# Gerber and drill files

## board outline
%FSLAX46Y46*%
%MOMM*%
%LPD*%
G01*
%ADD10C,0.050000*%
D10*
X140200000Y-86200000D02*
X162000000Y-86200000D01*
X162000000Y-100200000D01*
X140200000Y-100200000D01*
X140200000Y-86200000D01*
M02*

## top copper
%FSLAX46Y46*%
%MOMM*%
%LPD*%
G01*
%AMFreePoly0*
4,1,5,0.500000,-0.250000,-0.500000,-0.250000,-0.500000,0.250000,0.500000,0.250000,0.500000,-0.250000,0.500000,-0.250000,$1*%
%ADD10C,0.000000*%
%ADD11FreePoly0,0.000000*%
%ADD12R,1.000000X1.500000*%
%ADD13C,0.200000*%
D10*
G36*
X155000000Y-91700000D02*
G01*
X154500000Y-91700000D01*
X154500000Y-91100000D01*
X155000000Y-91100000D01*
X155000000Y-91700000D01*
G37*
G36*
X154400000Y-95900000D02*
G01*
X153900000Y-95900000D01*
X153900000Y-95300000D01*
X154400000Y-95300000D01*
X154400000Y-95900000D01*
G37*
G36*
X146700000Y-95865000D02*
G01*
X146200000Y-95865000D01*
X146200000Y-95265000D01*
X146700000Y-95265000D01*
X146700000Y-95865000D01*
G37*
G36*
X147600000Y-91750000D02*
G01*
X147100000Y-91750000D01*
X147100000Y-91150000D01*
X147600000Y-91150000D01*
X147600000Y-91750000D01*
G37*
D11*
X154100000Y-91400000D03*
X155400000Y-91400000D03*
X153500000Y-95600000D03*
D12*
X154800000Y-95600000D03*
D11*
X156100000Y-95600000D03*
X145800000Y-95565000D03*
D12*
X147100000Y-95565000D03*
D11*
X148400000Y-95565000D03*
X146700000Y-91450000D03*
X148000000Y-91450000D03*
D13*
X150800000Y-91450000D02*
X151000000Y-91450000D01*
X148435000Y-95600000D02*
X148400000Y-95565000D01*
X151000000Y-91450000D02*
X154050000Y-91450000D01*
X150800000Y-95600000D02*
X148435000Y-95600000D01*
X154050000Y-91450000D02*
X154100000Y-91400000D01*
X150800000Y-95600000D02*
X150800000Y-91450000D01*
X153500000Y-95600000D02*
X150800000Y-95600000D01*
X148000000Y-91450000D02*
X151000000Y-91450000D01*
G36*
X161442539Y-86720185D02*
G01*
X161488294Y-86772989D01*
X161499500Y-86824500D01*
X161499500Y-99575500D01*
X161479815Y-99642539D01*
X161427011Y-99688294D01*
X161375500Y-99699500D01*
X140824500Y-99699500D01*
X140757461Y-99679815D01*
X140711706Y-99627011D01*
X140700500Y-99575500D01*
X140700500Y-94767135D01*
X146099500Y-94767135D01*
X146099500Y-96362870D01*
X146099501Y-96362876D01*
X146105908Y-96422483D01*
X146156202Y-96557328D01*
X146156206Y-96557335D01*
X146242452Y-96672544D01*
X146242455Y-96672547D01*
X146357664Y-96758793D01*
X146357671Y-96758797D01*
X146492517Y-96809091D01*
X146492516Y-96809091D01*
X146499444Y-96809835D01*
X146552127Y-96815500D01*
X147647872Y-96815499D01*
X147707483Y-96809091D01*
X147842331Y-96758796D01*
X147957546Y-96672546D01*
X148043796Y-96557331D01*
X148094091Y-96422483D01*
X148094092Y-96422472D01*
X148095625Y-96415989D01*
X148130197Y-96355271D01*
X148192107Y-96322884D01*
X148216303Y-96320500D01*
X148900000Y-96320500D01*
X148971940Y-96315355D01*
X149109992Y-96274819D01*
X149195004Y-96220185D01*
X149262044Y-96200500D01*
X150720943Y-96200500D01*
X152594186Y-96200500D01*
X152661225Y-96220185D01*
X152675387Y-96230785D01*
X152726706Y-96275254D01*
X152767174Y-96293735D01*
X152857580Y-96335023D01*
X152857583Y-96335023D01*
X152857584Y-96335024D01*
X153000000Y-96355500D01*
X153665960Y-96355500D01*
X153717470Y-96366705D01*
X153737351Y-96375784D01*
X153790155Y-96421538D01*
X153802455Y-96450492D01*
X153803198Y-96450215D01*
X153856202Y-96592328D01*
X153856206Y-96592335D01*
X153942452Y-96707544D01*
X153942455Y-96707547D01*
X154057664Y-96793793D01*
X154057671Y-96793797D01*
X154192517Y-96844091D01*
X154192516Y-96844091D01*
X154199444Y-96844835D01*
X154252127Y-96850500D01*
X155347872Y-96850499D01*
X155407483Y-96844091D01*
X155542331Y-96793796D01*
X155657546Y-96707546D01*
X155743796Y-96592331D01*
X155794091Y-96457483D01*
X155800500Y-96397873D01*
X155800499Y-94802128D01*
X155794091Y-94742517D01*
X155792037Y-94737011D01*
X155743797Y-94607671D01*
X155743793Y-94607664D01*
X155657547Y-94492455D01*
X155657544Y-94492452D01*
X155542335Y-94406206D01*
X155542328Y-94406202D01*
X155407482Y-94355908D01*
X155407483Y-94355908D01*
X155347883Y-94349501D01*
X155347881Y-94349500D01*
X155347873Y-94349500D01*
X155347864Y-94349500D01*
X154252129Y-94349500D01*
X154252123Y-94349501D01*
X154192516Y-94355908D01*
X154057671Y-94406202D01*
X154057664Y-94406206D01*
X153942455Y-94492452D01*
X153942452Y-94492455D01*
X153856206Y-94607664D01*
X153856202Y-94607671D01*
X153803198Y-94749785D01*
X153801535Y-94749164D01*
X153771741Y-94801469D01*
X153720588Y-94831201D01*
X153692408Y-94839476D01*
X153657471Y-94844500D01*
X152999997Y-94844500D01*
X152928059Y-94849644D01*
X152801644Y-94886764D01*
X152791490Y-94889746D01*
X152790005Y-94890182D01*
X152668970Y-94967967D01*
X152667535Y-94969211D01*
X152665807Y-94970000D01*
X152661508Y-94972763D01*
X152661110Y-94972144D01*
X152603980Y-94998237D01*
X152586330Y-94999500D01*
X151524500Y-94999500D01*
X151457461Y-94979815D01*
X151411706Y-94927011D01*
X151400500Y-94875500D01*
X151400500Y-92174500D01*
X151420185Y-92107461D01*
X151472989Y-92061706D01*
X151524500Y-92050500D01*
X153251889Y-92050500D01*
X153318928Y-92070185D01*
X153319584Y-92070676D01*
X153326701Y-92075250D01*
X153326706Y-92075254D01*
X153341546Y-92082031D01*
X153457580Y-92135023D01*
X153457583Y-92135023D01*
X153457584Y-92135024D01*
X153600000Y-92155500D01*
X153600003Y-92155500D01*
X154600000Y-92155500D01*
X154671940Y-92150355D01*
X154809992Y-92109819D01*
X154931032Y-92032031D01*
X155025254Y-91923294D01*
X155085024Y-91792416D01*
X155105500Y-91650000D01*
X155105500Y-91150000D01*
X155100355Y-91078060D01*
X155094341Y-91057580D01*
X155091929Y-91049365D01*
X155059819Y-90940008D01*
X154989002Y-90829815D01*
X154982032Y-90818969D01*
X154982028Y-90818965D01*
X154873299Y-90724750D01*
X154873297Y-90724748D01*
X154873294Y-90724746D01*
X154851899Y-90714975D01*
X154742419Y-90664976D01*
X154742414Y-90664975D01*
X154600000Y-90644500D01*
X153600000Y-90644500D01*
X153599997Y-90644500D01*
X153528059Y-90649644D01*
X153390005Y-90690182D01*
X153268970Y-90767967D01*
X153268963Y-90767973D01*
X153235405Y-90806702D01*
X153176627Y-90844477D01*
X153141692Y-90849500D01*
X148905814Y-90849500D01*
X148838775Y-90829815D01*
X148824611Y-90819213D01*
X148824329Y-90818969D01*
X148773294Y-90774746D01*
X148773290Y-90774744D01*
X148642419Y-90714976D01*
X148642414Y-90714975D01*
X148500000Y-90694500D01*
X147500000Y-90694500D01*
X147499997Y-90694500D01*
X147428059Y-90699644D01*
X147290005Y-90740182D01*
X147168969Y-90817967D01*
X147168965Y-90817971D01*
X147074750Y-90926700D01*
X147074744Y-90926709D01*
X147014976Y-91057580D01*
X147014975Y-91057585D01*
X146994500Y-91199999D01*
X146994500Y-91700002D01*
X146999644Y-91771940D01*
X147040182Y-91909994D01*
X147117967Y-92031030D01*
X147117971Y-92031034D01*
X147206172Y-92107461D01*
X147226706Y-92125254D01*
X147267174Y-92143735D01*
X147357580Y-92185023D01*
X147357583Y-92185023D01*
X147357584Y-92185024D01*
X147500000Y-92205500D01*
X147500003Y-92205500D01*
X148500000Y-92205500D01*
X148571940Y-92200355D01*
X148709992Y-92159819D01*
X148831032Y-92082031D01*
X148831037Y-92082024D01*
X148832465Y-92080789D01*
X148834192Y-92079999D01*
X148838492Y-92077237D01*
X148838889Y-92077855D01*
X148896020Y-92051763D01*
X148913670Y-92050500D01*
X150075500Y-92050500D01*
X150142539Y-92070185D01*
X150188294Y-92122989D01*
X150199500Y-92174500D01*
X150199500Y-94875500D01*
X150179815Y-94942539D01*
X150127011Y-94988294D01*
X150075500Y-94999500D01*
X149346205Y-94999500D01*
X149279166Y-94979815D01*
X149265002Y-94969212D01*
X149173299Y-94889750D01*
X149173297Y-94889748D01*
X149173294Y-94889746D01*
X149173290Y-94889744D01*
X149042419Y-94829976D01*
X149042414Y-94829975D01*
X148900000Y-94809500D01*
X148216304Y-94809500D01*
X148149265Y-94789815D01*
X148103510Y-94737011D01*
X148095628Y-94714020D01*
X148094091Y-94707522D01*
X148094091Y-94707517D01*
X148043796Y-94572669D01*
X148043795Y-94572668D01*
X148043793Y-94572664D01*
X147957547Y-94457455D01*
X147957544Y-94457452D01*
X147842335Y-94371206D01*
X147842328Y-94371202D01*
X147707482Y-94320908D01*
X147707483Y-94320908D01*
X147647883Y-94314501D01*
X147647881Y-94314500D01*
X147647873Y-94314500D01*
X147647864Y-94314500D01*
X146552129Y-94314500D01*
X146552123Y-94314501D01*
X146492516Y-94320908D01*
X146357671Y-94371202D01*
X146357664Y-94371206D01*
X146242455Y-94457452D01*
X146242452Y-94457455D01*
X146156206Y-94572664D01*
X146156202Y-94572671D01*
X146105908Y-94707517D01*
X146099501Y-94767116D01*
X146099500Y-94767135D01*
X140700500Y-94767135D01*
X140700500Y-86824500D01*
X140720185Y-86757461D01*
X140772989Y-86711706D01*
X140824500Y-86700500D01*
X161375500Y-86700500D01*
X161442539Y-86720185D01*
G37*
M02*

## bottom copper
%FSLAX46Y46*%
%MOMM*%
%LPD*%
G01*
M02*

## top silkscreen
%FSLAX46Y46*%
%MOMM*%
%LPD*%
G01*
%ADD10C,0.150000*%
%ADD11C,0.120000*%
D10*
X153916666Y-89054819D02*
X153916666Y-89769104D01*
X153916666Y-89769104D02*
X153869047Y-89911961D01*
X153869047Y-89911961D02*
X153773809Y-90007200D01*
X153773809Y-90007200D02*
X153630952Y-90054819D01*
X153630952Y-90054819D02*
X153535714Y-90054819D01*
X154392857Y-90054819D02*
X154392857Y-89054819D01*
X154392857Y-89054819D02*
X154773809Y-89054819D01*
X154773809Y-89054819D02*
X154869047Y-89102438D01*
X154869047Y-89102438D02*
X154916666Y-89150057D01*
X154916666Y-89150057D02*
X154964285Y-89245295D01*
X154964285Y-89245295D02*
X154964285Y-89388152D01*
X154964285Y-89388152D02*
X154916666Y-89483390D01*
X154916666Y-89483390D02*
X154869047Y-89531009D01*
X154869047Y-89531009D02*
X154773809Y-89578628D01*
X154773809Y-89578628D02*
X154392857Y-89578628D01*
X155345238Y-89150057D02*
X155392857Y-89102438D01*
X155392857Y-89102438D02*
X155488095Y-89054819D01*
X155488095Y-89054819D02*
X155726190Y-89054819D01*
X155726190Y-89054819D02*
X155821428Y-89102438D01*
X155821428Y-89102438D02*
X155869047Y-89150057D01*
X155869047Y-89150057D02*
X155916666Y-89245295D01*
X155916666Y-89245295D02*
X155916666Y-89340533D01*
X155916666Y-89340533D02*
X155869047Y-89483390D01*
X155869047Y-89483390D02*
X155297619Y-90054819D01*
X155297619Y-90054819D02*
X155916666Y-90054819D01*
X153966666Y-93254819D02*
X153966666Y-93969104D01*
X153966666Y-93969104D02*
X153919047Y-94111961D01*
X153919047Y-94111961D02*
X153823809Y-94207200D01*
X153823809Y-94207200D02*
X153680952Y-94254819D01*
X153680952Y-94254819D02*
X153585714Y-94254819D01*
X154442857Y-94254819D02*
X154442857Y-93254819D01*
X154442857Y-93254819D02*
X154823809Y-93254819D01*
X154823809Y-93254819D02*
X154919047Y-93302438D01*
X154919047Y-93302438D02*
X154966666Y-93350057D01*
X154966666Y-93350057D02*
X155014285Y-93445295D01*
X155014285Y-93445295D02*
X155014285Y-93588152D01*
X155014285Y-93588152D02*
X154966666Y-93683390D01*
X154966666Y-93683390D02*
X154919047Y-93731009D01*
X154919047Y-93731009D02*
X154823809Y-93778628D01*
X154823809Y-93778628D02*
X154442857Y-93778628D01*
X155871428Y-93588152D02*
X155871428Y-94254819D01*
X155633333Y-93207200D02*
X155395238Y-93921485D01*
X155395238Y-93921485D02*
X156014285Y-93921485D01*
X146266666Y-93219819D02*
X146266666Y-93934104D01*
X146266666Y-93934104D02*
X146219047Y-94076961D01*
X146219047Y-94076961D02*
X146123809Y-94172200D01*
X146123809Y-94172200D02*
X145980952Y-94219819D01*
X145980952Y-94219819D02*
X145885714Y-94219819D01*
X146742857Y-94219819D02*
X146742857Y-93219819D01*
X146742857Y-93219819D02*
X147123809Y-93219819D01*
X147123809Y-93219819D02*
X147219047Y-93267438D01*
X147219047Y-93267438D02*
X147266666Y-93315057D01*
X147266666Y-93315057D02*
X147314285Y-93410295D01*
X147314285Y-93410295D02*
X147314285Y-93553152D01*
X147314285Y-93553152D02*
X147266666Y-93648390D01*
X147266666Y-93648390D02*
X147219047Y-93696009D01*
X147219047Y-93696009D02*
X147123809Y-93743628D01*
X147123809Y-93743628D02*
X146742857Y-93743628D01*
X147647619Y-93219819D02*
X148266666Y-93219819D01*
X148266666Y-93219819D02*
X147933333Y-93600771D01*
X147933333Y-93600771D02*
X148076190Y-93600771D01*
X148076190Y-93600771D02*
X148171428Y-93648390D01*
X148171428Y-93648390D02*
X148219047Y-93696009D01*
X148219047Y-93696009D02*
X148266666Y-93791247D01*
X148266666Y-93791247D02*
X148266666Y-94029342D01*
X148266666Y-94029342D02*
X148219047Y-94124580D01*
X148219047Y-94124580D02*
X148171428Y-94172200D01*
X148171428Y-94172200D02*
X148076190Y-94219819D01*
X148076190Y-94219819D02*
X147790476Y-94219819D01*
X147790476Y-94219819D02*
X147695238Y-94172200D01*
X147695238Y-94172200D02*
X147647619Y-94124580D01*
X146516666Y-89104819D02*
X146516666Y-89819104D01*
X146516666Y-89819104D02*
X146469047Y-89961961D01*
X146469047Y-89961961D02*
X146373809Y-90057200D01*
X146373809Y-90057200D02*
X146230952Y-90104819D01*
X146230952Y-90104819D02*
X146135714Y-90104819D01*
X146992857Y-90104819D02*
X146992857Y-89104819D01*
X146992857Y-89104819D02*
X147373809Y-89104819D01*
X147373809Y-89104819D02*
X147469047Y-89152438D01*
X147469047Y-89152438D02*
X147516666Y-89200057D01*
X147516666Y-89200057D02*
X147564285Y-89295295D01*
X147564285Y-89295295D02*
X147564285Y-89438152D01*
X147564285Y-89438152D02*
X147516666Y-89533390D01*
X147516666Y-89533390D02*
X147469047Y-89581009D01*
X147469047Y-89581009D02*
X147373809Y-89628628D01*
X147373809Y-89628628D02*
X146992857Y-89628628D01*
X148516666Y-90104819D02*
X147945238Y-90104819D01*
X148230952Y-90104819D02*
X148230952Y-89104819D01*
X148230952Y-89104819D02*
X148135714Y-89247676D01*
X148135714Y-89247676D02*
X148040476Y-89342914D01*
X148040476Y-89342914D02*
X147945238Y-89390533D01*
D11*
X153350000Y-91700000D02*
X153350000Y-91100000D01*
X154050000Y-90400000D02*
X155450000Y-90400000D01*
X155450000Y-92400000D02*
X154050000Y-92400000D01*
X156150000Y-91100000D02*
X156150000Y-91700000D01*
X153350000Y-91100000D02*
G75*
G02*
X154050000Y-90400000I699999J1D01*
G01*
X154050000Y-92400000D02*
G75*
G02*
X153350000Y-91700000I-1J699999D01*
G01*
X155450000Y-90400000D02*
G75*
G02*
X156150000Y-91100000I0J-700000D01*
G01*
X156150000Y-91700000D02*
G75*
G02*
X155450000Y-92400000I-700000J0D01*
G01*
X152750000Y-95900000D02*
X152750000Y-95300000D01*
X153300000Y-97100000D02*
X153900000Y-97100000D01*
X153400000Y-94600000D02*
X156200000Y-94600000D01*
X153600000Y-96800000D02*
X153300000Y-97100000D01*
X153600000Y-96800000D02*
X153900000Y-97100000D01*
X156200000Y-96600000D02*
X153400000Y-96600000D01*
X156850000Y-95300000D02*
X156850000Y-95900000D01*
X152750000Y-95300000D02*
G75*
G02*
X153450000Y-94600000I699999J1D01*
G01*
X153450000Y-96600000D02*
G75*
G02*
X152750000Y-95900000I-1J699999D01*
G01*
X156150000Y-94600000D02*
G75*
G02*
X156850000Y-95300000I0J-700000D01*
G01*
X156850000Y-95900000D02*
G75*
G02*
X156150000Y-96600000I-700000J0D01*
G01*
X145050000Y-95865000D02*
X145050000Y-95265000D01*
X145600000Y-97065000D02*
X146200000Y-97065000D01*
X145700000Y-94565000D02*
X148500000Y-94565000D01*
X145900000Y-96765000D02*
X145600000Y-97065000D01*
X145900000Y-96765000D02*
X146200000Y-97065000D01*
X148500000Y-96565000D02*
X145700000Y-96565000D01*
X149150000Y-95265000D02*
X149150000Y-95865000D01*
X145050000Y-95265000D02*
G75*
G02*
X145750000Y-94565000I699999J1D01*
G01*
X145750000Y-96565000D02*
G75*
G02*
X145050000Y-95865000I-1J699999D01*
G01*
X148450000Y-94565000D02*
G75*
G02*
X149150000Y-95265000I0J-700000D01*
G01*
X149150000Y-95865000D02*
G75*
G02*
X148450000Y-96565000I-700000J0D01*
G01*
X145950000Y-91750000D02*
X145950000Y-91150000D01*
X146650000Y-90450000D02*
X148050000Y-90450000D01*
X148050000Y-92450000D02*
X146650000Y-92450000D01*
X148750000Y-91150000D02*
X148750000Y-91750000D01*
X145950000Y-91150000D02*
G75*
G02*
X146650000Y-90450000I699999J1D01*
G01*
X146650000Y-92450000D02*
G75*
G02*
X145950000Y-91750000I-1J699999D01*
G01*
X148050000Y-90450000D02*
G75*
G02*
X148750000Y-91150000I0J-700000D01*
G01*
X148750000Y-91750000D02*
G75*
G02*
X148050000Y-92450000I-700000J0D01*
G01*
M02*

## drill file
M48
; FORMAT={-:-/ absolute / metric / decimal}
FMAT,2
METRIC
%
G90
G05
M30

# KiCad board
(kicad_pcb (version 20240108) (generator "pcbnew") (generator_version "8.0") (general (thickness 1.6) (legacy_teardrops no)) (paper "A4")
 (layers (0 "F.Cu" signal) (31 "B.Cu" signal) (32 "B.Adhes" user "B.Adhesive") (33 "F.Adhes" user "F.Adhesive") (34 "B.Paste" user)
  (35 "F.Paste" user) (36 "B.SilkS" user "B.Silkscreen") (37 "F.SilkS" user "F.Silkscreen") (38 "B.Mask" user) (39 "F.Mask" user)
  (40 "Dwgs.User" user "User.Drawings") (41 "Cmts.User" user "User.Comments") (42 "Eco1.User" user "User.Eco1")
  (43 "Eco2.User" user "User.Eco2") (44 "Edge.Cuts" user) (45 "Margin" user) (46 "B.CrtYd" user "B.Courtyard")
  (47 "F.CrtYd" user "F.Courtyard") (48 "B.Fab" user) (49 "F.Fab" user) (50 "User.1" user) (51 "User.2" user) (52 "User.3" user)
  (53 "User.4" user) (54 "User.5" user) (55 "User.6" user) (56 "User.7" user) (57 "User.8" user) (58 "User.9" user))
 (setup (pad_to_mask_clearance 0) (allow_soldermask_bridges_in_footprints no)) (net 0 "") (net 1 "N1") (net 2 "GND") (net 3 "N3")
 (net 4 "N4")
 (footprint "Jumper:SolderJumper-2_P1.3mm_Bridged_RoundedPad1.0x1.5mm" (layer "F.Cu") (at 154.75 91.4)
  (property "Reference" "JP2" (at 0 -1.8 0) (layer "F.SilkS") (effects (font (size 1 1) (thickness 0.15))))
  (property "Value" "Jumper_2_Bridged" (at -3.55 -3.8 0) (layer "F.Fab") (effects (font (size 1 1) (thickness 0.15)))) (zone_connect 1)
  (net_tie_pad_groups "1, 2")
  (fp_poly (pts (xy 0.25 -0.3) (xy -0.25 -0.3) (xy -0.25 0.3) (xy 0.25 0.3)) (stroke (width 0) (type solid)) (fill solid) (layer "F.Cu"))
  (fp_line (start -1.4 0.3) (end -1.4 -0.3) (stroke (width 0.12) (type solid)) (layer "F.SilkS"))
  (fp_line (start -0.7 -1) (end 0.7 -1) (stroke (width 0.12) (type solid)) (layer "F.SilkS"))
  (fp_line (start 0.7 1) (end -0.7 1) (stroke (width 0.12) (type solid)) (layer "F.SilkS"))
  (fp_line (start 1.4 -0.3) (end 1.4 0.3) (stroke (width 0.12) (type solid)) (layer "F.SilkS"))
  (fp_arc (start -1.4 -0.3) (mid -1.194975 -0.794975) (end -0.7 -1) (stroke (width 0.12) (type solid)) (layer "F.SilkS"))
  (fp_arc (start -0.7 1) (mid -1.194975 0.794975) (end -1.4 0.3) (stroke (width 0.12) (type solid)) (layer "F.SilkS"))
  (fp_arc (start 0.7 -1) (mid 1.194975 -0.794975) (end 1.4 -0.3) (stroke (width 0.12) (type solid)) (layer "F.SilkS"))
  (fp_arc (start 1.4 0.3) (mid 1.194975 0.794975) (end 0.7 1) (stroke (width 0.12) (type solid)) (layer "F.SilkS"))
  (pad "1" smd custom (at -0.65 0) (size 1 0.5) (layers "F.Cu" "F.Mask") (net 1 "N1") (zone_connect 2) (thermal_bridge_angle 45)
   (options (clearance outline) (anchor rect)) (primitives))
  (pad "2" smd custom (at 0.65 0) (size 1 0.5) (layers "F.Cu" "F.Mask") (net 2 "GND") (zone_connect 2) (thermal_bridge_angle 45)
   (options (clearance outline) (anchor rect)) (primitives)))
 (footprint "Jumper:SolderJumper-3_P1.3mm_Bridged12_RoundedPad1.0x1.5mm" (layer "F.Cu") (at 154.8 95.6)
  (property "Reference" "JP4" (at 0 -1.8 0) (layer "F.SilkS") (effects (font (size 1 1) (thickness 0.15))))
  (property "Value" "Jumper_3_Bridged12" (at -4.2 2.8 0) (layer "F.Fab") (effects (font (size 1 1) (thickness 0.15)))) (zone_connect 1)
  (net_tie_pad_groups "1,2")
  (fp_poly (pts (xy -0.9 -0.3) (xy -0.4 -0.3) (xy -0.4 0.3) (xy -0.9 0.3)) (stroke (width 0) (type solid)) (fill solid) (layer "F.Cu"))
  (fp_line (start -2.05 0.3) (end -2.05 -0.3) (stroke (width 0.12) (type solid)) (layer "F.SilkS"))
  (fp_line (start -1.5 1.5) (end -0.9 1.5) (stroke (width 0.12) (type solid)) (layer "F.SilkS"))
  (fp_line (start -1.4 -1) (end 1.4 -1) (stroke (width 0.12) (type solid)) (layer "F.SilkS"))
  (fp_line (start -1.2 1.2) (end -1.5 1.5) (stroke (width 0.12) (type solid)) (layer "F.SilkS"))
  (fp_line (start -1.2 1.2) (end -0.9 1.5) (stroke (width 0.12) (type solid)) (layer "F.SilkS"))
  (fp_line (start 1.4 1) (end -1.4 1) (stroke (width 0.12) (type solid)) (layer "F.SilkS"))
  (fp_line (start 2.05 -0.3) (end 2.05 0.3) (stroke (width 0.12) (type solid)) (layer "F.SilkS"))
  (fp_arc (start -2.05 -0.3) (mid -1.844975 -0.794975) (end -1.35 -1) (stroke (width 0.12) (type solid)) (layer "F.SilkS"))
  (fp_arc (start -1.35 1) (mid -1.844975 0.794975) (end -2.05 0.3) (stroke (width 0.12) (type solid)) (layer "F.SilkS"))
  (fp_arc (start 1.35 -1) (mid 1.844975 -0.794975) (end 2.05 -0.3) (stroke (width 0.12) (type solid)) (layer "F.SilkS"))
  (fp_arc (start 2.05 0.3) (mid 1.844975 0.794975) (end 1.35 1) (stroke (width 0.12) (type solid)) (layer "F.SilkS"))
  (pad "1" smd custom (at -1.3 0) (size 1 0.5) (layers "F.Cu" "F.Mask") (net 1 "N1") (zone_connect 2) (thermal_bridge_angle 45)
   (options (clearance outline) (anchor rect)) (primitives))
  (pad "2" smd rect (at 0 0) (size 1 1.5) (layers "F.Cu" "F.Mask") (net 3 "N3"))
  (pad "3" smd custom (at 1.3 0) (size 1 0.5) (layers "F.Cu" "F.Mask") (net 2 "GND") (zone_connect 2) (thermal_bridge_angle 45)
   (options (clearance outline) (anchor rect)) (primitives)))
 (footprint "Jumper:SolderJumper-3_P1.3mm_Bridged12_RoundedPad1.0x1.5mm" (layer "F.Cu") (at 147.1 95.565)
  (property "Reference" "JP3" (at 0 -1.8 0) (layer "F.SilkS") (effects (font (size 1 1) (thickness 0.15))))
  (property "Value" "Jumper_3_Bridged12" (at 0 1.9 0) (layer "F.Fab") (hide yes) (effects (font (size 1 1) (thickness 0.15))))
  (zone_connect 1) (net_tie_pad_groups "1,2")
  (fp_poly (pts (xy -0.9 -0.3) (xy -0.4 -0.3) (xy -0.4 0.3) (xy -0.9 0.3)) (stroke (width 0) (type solid)) (fill solid) (layer "F.Cu"))
  (fp_line (start -2.05 0.3) (end -2.05 -0.3) (stroke (width 0.12) (type solid)) (layer "F.SilkS"))
  (fp_line (start -1.5 1.5) (end -0.9 1.5) (stroke (width 0.12) (type solid)) (layer "F.SilkS"))
  (fp_line (start -1.4 -1) (end 1.4 -1) (stroke (width 0.12) (type solid)) (layer "F.SilkS"))
  (fp_line (start -1.2 1.2) (end -1.5 1.5) (stroke (width 0.12) (type solid)) (layer "F.SilkS"))
  (fp_line (start -1.2 1.2) (end -0.9 1.5) (stroke (width 0.12) (type solid)) (layer "F.SilkS"))
  (fp_line (start 1.4 1) (end -1.4 1) (stroke (width 0.12) (type solid)) (layer "F.SilkS"))
  (fp_line (start 2.05 -0.3) (end 2.05 0.3) (stroke (width 0.12) (type solid)) (layer "F.SilkS"))
  (fp_arc (start -2.05 -0.3) (mid -1.844975 -0.794975) (end -1.35 -1) (stroke (width 0.12) (type solid)) (layer "F.SilkS"))
  (fp_arc (start -1.35 1) (mid -1.844975 0.794975) (end -2.05 0.3) (stroke (width 0.12) (type solid)) (layer "F.SilkS"))
  (fp_arc (start 1.35 -1) (mid 1.844975 -0.794975) (end 2.05 -0.3) (stroke (width 0.12) (type solid)) (layer "F.SilkS"))
  (fp_arc (start 2.05 0.3) (mid 1.844975 0.794975) (end 1.35 1) (stroke (width 0.12) (type solid)) (layer "F.SilkS"))
  (pad "1" smd custom (at -1.3 0) (size 1 0.5) (layers "F.Cu" "F.Mask") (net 2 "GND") (zone_connect 2) (thermal_bridge_angle 45)
   (options (clearance outline) (anchor rect)) (primitives))
  (pad "2" smd rect (at 0 0) (size 1 1.5) (layers "F.Cu" "F.Mask") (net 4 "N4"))
  (pad "3" smd custom (at 1.3 0) (size 1 0.5) (layers "F.Cu" "F.Mask") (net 1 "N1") (zone_connect 2) (thermal_bridge_angle 45)
   (options (clearance outline) (anchor rect)) (primitives)))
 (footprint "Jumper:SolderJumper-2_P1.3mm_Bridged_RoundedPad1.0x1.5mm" (layer "F.Cu") (at 147.35 91.45)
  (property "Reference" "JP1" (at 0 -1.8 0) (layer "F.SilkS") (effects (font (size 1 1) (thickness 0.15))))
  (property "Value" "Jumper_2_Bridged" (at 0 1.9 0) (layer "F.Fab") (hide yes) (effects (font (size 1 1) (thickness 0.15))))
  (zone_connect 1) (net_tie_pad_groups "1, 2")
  (fp_poly (pts (xy 0.25 -0.3) (xy -0.25 -0.3) (xy -0.25 0.3) (xy 0.25 0.3)) (stroke (width 0) (type solid)) (fill solid) (layer "F.Cu"))
  (fp_line (start -1.4 0.3) (end -1.4 -0.3) (stroke (width 0.12) (type solid)) (layer "F.SilkS"))
  (fp_line (start -0.7 -1) (end 0.7 -1) (stroke (width 0.12) (type solid)) (layer "F.SilkS"))
  (fp_line (start 0.7 1) (end -0.7 1) (stroke (width 0.12) (type solid)) (layer "F.SilkS"))
  (fp_line (start 1.4 -0.3) (end 1.4 0.3) (stroke (width 0.12) (type solid)) (layer "F.SilkS"))
  (fp_arc (start -1.4 -0.3) (mid -1.194975 -0.794975) (end -0.7 -1) (stroke (width 0.12) (type solid)) (layer "F.SilkS"))
  (fp_arc (start -0.7 1) (mid -1.194975 0.794975) (end -1.4 0.3) (stroke (width 0.12) (type solid)) (layer "F.SilkS"))
  (fp_arc (start 0.7 -1) (mid 1.194975 -0.794975) (end 1.4 -0.3) (stroke (width 0.12) (type solid)) (layer "F.SilkS"))
  (fp_arc (start 1.4 0.3) (mid 1.194975 0.794975) (end 0.7 1) (stroke (width 0.12) (type solid)) (layer "F.SilkS"))
  (pad "1" smd custom (at -0.65 0) (size 1 0.5) (layers "F.Cu" "F.Mask") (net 2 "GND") (zone_connect 2) (thermal_bridge_angle 45)
   (options (clearance outline) (anchor rect)) (primitives))
  (pad "2" smd custom (at 0.65 0) (size 1 0.5) (layers "F.Cu" "F.Mask") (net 1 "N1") (zone_connect 2) (thermal_bridge_angle 45)
   (options (clearance outline) (anchor rect)) (primitives)))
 (gr_rect (start 140.2 86.2) (end 162 100.2) (stroke (width 0.05) (type default)) (fill none) (layer "Edge.Cuts"))
 (segment (start 150.8 91.45) (end 151 91.45) (width 0.2) (layer "F.Cu") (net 1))
 (segment (start 148.435 95.6) (end 148.4 95.565) (width 0.2) (layer "F.Cu") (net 1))
 (segment (start 151 91.45) (end 154.05 91.45) (width 0.2) (layer "F.Cu") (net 1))
 (segment (start 150.8 95.6) (end 148.435 95.6) (width 0.2) (layer "F.Cu") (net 1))
 (segment (start 154.05 91.45) (end 154.1 91.4) (width 0.2) (layer "F.Cu") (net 1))
 (segment (start 150.8 95.6) (end 150.8 91.45) (width 0.2) (layer "F.Cu") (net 1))
 (segment (start 153.5 95.6) (end 150.8 95.6) (width 0.2) (layer "F.Cu") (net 1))
 (segment (start 148 91.45) (end 151 91.45) (width 0.2) (layer "F.Cu") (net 1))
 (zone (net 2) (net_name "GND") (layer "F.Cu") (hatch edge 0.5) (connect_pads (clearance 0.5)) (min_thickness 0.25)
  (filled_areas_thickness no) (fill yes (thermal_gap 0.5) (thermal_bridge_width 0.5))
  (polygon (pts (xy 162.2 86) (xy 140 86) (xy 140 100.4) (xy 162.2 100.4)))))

